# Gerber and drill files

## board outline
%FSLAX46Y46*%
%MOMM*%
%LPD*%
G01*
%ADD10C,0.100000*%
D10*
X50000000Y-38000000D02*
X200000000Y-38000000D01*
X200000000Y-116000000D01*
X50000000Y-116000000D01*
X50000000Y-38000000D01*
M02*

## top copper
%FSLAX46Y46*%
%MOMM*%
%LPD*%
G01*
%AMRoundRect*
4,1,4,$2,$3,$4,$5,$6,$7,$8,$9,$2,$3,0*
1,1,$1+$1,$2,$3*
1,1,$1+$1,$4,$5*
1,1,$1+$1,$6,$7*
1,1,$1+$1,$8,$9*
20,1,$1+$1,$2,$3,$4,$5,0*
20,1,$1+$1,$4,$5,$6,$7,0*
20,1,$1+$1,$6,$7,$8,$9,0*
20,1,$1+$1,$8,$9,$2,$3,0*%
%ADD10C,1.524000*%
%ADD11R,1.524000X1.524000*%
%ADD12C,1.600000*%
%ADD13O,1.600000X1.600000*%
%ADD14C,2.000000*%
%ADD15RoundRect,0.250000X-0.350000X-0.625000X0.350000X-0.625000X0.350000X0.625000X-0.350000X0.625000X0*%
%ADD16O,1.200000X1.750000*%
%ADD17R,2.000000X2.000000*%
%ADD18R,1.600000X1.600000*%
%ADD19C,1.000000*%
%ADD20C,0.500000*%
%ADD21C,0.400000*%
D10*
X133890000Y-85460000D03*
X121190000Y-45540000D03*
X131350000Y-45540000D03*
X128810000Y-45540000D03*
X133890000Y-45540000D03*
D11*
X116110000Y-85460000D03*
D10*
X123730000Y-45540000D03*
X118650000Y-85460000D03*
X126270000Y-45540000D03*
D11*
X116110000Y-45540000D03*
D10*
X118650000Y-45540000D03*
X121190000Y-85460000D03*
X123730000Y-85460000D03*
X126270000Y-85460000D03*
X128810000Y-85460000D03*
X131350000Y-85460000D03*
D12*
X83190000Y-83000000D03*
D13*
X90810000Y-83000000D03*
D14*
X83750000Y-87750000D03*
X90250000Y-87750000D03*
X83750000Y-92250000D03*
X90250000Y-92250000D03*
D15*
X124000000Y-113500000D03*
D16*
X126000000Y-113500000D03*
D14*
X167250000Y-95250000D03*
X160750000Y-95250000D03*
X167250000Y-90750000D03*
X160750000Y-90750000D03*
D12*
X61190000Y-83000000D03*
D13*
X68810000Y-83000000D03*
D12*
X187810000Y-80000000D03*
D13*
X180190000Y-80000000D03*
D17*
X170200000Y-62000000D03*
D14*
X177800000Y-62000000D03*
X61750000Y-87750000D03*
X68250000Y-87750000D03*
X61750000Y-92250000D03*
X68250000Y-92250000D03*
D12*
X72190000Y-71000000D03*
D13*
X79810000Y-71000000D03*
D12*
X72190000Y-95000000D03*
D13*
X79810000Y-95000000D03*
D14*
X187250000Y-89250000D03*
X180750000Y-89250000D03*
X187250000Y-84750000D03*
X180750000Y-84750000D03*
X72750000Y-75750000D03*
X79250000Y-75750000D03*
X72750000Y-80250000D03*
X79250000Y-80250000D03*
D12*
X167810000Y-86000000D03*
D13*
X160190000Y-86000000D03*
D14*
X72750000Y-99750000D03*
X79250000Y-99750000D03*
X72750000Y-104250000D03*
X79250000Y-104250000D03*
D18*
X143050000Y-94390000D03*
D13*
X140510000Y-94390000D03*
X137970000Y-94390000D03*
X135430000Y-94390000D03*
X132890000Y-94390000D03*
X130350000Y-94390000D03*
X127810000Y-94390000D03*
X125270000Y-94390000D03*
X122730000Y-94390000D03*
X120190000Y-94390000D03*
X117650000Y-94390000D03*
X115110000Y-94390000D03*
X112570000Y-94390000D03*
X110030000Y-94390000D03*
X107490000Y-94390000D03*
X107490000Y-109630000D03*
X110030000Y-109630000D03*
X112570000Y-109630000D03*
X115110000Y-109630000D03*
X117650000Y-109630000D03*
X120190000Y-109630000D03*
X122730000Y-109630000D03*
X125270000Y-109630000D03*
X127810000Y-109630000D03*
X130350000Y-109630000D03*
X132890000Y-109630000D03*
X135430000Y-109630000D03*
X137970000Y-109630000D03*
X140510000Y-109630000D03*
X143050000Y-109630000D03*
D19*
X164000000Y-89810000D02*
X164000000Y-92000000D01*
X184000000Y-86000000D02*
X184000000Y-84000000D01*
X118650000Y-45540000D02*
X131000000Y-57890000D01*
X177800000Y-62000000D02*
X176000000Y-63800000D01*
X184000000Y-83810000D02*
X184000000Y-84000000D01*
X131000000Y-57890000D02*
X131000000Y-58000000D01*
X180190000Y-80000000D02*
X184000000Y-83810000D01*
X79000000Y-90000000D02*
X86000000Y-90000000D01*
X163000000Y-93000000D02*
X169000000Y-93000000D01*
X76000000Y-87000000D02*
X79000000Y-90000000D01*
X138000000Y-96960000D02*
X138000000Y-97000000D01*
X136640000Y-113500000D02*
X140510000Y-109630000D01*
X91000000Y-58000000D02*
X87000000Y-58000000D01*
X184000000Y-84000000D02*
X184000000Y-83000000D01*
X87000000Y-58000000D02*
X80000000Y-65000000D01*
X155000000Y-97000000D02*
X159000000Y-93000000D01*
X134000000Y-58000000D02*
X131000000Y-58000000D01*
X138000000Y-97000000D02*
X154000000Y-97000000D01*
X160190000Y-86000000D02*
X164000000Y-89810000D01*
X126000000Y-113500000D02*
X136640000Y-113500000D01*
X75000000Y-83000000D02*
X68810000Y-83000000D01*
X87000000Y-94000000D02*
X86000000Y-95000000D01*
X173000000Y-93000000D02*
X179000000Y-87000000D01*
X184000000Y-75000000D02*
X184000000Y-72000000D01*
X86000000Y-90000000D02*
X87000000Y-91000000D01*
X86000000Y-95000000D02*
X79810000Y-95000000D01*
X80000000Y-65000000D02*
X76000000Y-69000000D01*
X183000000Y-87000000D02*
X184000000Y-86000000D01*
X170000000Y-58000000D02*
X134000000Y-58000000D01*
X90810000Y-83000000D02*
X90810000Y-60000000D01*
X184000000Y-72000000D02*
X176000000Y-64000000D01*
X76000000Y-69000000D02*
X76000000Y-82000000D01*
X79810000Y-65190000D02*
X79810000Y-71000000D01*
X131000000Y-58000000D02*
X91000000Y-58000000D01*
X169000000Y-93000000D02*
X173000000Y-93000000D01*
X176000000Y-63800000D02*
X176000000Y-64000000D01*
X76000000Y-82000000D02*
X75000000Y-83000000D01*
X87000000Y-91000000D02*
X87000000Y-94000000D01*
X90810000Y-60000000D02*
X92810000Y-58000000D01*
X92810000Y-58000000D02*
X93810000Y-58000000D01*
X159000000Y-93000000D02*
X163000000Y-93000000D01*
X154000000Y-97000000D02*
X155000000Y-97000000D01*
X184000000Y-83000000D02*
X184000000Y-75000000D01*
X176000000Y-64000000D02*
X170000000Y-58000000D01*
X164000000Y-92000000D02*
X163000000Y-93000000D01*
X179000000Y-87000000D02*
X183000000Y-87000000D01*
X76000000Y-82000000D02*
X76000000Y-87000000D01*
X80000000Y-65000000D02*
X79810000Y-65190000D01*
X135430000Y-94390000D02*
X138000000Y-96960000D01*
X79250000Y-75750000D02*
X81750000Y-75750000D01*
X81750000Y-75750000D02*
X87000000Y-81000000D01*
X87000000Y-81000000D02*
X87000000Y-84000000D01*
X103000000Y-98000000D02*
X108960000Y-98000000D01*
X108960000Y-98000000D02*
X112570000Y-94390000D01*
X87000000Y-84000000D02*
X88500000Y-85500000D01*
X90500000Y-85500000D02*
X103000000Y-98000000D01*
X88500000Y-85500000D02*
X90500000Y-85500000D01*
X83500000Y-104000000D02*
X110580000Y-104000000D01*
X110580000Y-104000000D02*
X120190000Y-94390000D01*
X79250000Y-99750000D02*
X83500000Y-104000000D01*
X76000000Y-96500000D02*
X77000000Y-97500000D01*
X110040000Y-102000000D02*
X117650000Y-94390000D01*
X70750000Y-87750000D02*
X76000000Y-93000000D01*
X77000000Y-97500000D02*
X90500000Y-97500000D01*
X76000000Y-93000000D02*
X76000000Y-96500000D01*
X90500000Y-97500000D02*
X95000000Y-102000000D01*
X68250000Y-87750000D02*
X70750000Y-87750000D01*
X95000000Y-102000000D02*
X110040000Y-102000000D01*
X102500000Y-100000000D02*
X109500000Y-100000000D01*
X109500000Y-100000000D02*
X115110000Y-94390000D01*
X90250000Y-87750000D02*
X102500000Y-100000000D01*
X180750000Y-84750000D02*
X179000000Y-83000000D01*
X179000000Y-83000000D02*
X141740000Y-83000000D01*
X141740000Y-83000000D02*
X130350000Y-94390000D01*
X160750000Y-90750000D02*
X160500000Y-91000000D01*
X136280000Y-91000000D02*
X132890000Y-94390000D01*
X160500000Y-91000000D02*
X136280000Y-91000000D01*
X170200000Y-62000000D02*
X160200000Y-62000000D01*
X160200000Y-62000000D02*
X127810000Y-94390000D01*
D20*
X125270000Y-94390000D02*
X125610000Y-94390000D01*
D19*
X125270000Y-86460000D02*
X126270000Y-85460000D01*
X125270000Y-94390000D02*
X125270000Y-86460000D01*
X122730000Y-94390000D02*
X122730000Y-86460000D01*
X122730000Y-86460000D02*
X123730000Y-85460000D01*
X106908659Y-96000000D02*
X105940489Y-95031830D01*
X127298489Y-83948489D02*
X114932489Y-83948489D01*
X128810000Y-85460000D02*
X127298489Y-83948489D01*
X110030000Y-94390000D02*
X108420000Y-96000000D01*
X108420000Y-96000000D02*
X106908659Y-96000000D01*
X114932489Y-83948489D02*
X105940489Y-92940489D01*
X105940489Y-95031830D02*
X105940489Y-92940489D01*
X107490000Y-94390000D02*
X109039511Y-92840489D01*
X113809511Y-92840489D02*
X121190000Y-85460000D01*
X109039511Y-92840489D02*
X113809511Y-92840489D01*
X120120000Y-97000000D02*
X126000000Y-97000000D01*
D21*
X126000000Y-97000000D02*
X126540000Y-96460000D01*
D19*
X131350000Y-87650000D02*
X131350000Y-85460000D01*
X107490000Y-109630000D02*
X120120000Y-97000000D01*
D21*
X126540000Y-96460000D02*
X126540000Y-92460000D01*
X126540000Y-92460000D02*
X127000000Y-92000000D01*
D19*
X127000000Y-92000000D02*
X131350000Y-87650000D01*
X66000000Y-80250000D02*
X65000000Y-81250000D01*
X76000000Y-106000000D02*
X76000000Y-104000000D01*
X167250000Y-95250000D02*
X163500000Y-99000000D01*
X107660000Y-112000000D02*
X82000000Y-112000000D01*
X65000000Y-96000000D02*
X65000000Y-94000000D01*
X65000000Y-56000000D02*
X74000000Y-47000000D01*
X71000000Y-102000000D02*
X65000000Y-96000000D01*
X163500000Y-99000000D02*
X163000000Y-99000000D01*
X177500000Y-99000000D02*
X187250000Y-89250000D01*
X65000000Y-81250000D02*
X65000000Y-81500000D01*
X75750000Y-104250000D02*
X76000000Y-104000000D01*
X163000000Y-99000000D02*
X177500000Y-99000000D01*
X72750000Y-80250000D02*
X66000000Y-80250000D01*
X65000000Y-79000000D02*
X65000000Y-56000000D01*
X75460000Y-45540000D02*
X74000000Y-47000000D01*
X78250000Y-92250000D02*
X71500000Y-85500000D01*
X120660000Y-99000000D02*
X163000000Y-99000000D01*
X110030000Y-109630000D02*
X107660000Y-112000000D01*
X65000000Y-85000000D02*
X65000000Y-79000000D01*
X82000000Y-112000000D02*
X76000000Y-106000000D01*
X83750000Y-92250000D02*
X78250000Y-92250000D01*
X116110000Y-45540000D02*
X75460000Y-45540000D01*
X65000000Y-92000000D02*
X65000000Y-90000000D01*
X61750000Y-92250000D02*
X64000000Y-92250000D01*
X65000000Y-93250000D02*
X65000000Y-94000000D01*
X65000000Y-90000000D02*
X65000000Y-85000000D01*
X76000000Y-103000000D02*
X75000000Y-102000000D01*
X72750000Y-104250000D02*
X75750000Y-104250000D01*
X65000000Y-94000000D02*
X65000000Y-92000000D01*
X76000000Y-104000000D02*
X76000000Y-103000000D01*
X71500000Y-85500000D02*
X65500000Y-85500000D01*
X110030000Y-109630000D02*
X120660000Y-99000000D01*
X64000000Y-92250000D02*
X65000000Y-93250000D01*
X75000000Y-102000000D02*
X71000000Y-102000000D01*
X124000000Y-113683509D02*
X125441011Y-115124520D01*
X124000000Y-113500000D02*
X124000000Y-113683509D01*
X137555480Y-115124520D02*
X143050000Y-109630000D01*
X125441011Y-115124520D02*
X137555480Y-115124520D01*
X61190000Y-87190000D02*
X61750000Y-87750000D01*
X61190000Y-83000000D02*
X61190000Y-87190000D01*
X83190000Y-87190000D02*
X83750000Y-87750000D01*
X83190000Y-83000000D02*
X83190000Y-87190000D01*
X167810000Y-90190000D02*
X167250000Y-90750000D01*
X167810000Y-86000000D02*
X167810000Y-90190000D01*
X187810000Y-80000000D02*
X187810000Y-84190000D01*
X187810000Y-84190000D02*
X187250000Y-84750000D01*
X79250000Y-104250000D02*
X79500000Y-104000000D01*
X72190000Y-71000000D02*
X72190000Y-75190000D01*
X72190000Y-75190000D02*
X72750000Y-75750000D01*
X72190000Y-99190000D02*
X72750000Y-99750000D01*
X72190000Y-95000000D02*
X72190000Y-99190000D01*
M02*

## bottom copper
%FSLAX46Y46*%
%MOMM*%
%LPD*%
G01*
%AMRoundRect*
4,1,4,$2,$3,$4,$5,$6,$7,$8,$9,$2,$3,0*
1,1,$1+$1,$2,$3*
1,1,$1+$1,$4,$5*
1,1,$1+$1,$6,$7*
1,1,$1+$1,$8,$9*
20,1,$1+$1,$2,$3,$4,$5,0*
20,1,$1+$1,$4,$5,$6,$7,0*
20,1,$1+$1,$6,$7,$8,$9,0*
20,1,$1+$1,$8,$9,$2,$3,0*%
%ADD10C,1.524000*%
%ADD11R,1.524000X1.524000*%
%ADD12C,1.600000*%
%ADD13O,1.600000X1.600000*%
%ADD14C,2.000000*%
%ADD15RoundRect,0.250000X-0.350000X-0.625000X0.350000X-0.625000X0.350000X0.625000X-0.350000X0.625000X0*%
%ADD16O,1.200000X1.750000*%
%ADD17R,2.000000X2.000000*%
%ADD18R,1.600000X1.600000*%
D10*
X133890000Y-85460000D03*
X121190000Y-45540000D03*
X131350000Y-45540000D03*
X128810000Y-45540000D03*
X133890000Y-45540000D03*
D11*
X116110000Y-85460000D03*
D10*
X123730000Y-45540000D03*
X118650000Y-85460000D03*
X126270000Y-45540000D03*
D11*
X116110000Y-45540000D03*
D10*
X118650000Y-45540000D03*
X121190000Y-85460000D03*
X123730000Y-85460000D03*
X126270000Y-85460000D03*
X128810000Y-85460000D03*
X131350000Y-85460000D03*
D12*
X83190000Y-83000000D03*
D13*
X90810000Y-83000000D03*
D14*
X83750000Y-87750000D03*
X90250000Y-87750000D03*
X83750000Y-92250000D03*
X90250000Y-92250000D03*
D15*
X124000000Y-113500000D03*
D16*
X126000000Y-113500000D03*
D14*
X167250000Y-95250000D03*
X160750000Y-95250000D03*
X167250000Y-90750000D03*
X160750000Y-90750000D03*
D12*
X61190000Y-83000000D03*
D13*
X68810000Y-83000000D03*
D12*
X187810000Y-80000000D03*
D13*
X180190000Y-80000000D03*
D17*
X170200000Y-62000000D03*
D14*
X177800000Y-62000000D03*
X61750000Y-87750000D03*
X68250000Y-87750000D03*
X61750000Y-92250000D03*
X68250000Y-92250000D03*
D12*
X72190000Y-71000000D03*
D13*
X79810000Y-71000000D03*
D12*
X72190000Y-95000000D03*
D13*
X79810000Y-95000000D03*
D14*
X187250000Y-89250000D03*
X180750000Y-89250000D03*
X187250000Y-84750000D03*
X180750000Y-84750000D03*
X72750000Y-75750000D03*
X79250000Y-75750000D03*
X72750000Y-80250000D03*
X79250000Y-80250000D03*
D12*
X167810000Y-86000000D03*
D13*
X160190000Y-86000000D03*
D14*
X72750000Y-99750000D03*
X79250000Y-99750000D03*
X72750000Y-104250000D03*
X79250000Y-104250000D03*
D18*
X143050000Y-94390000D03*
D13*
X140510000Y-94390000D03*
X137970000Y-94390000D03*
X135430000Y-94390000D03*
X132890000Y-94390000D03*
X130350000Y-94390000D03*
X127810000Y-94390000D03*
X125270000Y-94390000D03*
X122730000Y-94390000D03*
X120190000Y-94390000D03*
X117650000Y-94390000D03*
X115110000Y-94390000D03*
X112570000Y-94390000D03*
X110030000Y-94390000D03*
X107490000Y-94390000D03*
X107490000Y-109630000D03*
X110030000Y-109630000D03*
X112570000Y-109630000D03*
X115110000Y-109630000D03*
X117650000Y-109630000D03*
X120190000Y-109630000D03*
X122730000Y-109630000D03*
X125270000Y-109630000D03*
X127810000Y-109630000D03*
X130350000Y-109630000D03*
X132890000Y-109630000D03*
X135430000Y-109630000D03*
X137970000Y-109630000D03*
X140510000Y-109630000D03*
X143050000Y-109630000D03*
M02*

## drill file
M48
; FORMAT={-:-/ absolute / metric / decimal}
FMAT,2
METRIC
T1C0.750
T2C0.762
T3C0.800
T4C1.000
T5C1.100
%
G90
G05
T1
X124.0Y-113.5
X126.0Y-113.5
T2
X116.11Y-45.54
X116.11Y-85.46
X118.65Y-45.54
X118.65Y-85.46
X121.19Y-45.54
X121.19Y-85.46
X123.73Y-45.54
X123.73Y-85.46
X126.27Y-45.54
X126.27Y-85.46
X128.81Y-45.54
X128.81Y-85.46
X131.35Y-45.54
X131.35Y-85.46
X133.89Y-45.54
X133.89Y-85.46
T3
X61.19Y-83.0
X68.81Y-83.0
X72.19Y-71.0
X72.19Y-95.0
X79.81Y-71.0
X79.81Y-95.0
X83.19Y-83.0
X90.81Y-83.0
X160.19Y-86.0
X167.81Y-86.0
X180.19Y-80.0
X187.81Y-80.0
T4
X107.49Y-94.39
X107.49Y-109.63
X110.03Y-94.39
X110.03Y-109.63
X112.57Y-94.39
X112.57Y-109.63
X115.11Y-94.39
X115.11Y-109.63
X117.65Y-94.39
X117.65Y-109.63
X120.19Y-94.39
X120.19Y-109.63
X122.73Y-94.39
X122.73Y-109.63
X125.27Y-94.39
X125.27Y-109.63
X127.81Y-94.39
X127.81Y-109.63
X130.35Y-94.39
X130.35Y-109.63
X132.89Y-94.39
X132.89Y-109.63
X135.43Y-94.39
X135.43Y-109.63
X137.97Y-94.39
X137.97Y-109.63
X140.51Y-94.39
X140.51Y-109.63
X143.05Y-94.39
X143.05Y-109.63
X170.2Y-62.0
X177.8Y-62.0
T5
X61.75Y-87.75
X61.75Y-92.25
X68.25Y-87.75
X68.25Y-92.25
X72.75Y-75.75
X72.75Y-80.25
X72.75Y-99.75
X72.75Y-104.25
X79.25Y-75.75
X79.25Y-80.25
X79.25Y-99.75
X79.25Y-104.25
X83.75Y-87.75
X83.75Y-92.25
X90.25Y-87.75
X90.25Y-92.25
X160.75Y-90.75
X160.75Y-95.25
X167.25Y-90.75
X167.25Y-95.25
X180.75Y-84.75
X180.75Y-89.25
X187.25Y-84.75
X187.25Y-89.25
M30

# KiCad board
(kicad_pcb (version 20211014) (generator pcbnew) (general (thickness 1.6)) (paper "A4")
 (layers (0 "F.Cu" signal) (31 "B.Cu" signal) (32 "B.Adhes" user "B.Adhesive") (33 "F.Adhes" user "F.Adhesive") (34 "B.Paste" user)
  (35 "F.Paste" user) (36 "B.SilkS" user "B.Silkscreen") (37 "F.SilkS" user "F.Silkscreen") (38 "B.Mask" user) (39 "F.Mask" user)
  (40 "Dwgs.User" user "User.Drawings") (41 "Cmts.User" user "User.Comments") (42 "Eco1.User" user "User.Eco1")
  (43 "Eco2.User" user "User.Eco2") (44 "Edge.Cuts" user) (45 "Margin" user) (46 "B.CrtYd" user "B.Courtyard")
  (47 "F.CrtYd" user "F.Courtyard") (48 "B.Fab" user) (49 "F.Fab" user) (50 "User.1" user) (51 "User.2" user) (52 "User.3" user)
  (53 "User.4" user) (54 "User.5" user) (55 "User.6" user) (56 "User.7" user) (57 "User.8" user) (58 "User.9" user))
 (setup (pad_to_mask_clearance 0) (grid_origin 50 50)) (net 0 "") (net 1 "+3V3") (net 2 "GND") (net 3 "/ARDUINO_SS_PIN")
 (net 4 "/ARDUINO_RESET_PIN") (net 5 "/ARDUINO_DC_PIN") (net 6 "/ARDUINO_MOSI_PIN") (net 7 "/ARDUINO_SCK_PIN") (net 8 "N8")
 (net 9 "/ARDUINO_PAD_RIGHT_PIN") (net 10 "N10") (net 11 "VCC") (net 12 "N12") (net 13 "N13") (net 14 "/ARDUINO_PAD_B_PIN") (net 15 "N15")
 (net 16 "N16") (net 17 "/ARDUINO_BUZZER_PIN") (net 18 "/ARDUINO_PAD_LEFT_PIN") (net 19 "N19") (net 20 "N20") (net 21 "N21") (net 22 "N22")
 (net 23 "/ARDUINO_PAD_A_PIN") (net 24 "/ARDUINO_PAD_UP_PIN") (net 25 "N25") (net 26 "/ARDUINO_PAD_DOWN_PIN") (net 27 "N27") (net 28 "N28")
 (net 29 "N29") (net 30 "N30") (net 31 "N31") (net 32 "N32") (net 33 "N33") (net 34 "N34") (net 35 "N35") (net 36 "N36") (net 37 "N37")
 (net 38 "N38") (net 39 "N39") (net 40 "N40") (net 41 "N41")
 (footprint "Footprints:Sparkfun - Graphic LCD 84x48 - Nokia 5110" (layer "F.Cu") (at 125 43)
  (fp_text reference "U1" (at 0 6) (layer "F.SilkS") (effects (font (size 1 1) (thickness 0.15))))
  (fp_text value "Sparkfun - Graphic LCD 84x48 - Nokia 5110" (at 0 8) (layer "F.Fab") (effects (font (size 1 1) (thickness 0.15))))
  (pad "" thru_hole circle (at 8.89 42.46) (size 1.524 1.524) (drill 0.762) (layers *.Cu *.Mask))
  (pad "" thru_hole circle (at -3.81 2.54) (size 1.524 1.524) (drill 0.762) (layers *.Cu *.Mask))
  (pad "" thru_hole circle (at 6.35 2.54) (size 1.524 1.524) (drill 0.762) (layers *.Cu *.Mask))
  (pad "" thru_hole circle (at 3.81 2.54) (size 1.524 1.524) (drill 0.762) (layers *.Cu *.Mask))
  (pad "" thru_hole circle (at 8.89 2.54) (size 1.524 1.524) (drill 0.762) (layers *.Cu *.Mask))
  (pad "" thru_hole rect (at -8.89 42.46) (size 1.524 1.524) (drill 0.762) (layers *.Cu *.Mask))
  (pad "" thru_hole circle (at -1.27 2.54) (size 1.524 1.524) (drill 0.762) (layers *.Cu *.Mask))
  (pad "" thru_hole circle (at -6.35 42.46) (size 1.524 1.524) (drill 0.762) (layers *.Cu *.Mask))
  (pad "" thru_hole circle (at 1.27 2.54) (size 1.524 1.524) (drill 0.762) (layers *.Cu *.Mask))
  (pad "1" thru_hole rect (at -8.89 2.54) (size 1.524 1.524) (drill 0.762) (layers *.Cu *.Mask) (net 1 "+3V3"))
  (pad "2" thru_hole circle (at -6.35 2.54) (size 1.524 1.524) (drill 0.762) (layers *.Cu *.Mask) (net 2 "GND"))
  (pad "3" thru_hole circle (at -3.81 42.46) (size 1.524 1.524) (drill 0.762) (layers *.Cu *.Mask) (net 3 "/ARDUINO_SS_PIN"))
  (pad "4" thru_hole circle (at -1.27 42.46) (size 1.524 1.524) (drill 0.762) (layers *.Cu *.Mask) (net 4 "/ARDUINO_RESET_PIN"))
  (pad "5" thru_hole circle (at 1.27 42.46) (size 1.524 1.524) (drill 0.762) (layers *.Cu *.Mask) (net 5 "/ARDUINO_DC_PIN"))
  (pad "6" thru_hole circle (at 3.81 42.46) (size 1.524 1.524) (drill 0.762) (layers *.Cu *.Mask) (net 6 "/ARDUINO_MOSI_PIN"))
  (pad "7" thru_hole circle (at 6.35 42.46) (size 1.524 1.524) (drill 0.762) (layers *.Cu *.Mask) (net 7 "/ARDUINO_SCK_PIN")))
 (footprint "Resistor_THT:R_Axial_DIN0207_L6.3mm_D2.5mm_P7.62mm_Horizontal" (layer "F.Cu") (at 83.19 83)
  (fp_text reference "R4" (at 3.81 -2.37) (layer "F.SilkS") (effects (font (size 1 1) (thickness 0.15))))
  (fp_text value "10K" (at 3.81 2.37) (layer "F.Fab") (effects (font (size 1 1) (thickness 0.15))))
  (pad "1" thru_hole circle (at 0 0) (size 1.6 1.6) (drill 0.8) (layers *.Cu *.Mask) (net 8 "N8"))
  (pad "2" thru_hole oval (at 7.62 0) (size 1.6 1.6) (drill 0.8) (layers *.Cu *.Mask) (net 2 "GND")))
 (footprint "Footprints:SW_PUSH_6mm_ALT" (layer "F.Cu") (at 83.75 87.75)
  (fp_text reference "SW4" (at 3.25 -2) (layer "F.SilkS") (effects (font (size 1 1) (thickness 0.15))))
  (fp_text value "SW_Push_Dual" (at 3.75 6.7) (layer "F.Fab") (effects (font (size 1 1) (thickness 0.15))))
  (pad "1" thru_hole circle (at 0 0 90) (size 2 2) (drill 1.1) (layers *.Cu *.Mask) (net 8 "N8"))
  (pad "2" thru_hole circle (at 6.5 0 90) (size 2 2) (drill 1.1) (layers *.Cu *.Mask) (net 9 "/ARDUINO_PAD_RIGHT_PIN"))
  (pad "3" thru_hole circle (at 0 4.5 90) (size 2 2) (drill 1.1) (layers *.Cu *.Mask) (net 1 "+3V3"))
  (pad "4" thru_hole circle (at 6.5 4.5 90) (size 2 2) (drill 1.1) (layers *.Cu *.Mask) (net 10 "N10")))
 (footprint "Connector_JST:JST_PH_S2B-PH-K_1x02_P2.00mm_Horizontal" (layer "F.Cu") (at 124 113.5)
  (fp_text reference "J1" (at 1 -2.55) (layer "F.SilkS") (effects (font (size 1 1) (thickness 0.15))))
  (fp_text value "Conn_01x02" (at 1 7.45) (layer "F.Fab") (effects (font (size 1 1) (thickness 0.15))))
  (pad "1" thru_hole roundrect (at 0 0) (size 1.2 1.75) (drill 0.75) (layers *.Cu *.Mask) (roundrect_rratio 0.208333) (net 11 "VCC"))
  (pad "2" thru_hole oval (at 2 0) (size 1.2 1.75) (drill 0.75) (layers *.Cu *.Mask) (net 2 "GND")))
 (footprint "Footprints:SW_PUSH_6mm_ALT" (layer "F.Cu") (at 167.25 95.25 180)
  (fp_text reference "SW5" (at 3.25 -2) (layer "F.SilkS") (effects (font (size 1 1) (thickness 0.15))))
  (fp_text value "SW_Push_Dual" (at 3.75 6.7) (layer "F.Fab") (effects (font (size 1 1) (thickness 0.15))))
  (pad "1" thru_hole circle (at 0 0 270) (size 2 2) (drill 1.1) (layers *.Cu *.Mask) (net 1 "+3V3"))
  (pad "2" thru_hole circle (at 6.5 0 270) (size 2 2) (drill 1.1) (layers *.Cu *.Mask) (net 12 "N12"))
  (pad "3" thru_hole circle (at 0 4.5 270) (size 2 2) (drill 1.1) (layers *.Cu *.Mask) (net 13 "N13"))
  (pad "4" thru_hole circle (at 6.5 4.5 270) (size 2 2) (drill 1.1) (layers *.Cu *.Mask) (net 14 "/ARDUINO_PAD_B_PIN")))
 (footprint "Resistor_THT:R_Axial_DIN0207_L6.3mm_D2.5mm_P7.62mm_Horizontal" (layer "F.Cu") (at 61.19 83)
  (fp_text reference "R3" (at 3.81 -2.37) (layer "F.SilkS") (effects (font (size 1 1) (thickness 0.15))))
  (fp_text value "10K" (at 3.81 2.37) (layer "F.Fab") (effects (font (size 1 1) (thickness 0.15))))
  (pad "1" thru_hole circle (at 0 0) (size 1.6 1.6) (drill 0.8) (layers *.Cu *.Mask) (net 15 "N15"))
  (pad "2" thru_hole oval (at 7.62 0) (size 1.6 1.6) (drill 0.8) (layers *.Cu *.Mask) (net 2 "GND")))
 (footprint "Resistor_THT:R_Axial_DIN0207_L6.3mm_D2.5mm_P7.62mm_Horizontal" (layer "F.Cu") (at 187.81 80 180)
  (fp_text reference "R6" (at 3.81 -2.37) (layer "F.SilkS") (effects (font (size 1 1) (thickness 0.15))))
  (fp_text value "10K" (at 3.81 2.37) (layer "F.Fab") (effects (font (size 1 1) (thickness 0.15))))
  (pad "1" thru_hole circle (at 0 0 180) (size 1.6 1.6) (drill 0.8) (layers *.Cu *.Mask) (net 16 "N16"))
  (pad "2" thru_hole oval (at 7.62 0 180) (size 1.6 1.6) (drill 0.8) (layers *.Cu *.Mask) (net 2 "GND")))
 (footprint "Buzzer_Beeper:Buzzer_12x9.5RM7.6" (layer "F.Cu") (at 170.2 62)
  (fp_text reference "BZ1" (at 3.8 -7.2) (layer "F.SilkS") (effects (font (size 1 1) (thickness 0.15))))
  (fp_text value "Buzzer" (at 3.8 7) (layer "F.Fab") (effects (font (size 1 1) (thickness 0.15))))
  (pad "1" thru_hole rect (at 0 0) (size 2 2) (drill 1) (layers *.Cu *.Mask) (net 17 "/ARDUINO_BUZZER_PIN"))
  (pad "2" thru_hole circle (at 7.6 0) (size 2 2) (drill 1) (layers *.Cu *.Mask) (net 2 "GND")))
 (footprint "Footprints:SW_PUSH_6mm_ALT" (layer "F.Cu") (at 61.75 87.75)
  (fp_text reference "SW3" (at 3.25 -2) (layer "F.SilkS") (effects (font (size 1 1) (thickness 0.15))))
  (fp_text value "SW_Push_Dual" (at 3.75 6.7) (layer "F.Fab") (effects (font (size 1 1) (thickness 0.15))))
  (pad "1" thru_hole circle (at 0 0 90) (size 2 2) (drill 1.1) (layers *.Cu *.Mask) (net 15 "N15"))
  (pad "2" thru_hole circle (at 6.5 0 90) (size 2 2) (drill 1.1) (layers *.Cu *.Mask) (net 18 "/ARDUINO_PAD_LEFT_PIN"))
  (pad "3" thru_hole circle (at 0 4.5 90) (size 2 2) (drill 1.1) (layers *.Cu *.Mask) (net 1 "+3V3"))
  (pad "4" thru_hole circle (at 6.5 4.5 90) (size 2 2) (drill 1.1) (layers *.Cu *.Mask) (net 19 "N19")))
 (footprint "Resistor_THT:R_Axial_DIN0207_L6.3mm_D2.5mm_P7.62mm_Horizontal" (layer "F.Cu") (at 72.19 71)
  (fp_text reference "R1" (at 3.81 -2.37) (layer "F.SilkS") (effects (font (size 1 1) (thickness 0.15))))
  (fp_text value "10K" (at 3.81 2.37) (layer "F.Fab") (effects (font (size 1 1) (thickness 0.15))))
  (pad "1" thru_hole circle (at 0 0) (size 1.6 1.6) (drill 0.8) (layers *.Cu *.Mask) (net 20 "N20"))
  (pad "2" thru_hole oval (at 7.62 0) (size 1.6 1.6) (drill 0.8) (layers *.Cu *.Mask) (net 2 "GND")))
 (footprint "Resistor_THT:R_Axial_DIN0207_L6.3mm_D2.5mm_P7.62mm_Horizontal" (layer "F.Cu") (at 72.19 95)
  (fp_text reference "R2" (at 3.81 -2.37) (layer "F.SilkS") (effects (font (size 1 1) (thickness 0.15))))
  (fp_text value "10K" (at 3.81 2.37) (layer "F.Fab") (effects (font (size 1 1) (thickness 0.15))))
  (pad "1" thru_hole circle (at 0 0) (size 1.6 1.6) (drill 0.8) (layers *.Cu *.Mask) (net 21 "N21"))
  (pad "2" thru_hole oval (at 7.62 0) (size 1.6 1.6) (drill 0.8) (layers *.Cu *.Mask) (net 2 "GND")))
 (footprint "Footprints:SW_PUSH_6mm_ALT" (layer "F.Cu") (at 187.25 89.25 180)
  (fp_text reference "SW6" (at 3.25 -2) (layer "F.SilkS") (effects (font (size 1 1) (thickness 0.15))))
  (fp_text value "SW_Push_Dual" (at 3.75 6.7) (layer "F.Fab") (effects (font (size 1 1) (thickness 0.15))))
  (pad "1" thru_hole circle (at 0 0 270) (size 2 2) (drill 1.1) (layers *.Cu *.Mask) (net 1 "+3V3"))
  (pad "2" thru_hole circle (at 6.5 0 270) (size 2 2) (drill 1.1) (layers *.Cu *.Mask) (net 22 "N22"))
  (pad "3" thru_hole circle (at 0 4.5 270) (size 2 2) (drill 1.1) (layers *.Cu *.Mask) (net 16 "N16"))
  (pad "4" thru_hole circle (at 6.5 4.5 270) (size 2 2) (drill 1.1) (layers *.Cu *.Mask) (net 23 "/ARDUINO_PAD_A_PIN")))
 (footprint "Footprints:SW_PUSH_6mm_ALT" (layer "F.Cu") (at 72.75 75.75)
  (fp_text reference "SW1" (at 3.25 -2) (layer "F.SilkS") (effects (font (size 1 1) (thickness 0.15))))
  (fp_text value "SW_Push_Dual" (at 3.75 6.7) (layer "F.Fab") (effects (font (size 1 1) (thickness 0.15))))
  (pad "1" thru_hole circle (at 0 0 90) (size 2 2) (drill 1.1) (layers *.Cu *.Mask) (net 20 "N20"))
  (pad "2" thru_hole circle (at 6.5 0 90) (size 2 2) (drill 1.1) (layers *.Cu *.Mask) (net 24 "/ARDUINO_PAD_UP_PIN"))
  (pad "3" thru_hole circle (at 0 4.5 90) (size 2 2) (drill 1.1) (layers *.Cu *.Mask) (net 1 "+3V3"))
  (pad "4" thru_hole circle (at 6.5 4.5 90) (size 2 2) (drill 1.1) (layers *.Cu *.Mask) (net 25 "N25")))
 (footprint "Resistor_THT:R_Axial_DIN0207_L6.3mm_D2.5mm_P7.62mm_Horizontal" (layer "F.Cu") (at 167.81 86 180)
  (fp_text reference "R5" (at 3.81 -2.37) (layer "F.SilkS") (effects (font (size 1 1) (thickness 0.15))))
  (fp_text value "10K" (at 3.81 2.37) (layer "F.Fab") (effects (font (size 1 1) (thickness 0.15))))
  (pad "1" thru_hole circle (at 0 0 180) (size 1.6 1.6) (drill 0.8) (layers *.Cu *.Mask) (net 13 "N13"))
  (pad "2" thru_hole oval (at 7.62 0 180) (size 1.6 1.6) (drill 0.8) (layers *.Cu *.Mask) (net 2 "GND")))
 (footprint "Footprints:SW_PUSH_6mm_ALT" (layer "F.Cu") (at 72.75 99.75)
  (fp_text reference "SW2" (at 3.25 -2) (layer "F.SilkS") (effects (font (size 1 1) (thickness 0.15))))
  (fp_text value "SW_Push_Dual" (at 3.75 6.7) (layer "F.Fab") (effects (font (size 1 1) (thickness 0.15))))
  (pad "1" thru_hole circle (at 0 0 90) (size 2 2) (drill 1.1) (layers *.Cu *.Mask) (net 21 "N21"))
  (pad "2" thru_hole circle (at 6.5 0 90) (size 2 2) (drill 1.1) (layers *.Cu *.Mask) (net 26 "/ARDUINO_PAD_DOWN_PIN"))
  (pad "3" thru_hole circle (at 0 4.5 90) (size 2 2) (drill 1.1) (layers *.Cu *.Mask) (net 1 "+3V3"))
  (pad "4" thru_hole circle (at 6.5 4.5 90) (size 2 2) (drill 1.1) (layers *.Cu *.Mask) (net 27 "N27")))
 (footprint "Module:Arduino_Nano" (layer "F.Cu") (at 143.05 94.39 -90)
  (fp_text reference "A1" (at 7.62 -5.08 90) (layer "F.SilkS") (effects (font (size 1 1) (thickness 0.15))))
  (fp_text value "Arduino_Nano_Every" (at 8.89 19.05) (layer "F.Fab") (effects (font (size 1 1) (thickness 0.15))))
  (pad "1" thru_hole rect (at 0 0 270) (size 1.6 1.6) (drill 1) (layers *.Cu *.Mask) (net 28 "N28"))
  (pad "2" thru_hole oval (at 0 2.54 270) (size 1.6 1.6) (drill 1) (layers *.Cu *.Mask) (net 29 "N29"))
  (pad "3" thru_hole oval (at 0 5.08 270) (size 1.6 1.6) (drill 1) (layers *.Cu *.Mask) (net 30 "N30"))
  (pad "4" thru_hole oval (at 0 7.62 270) (size 1.6 1.6) (drill 1) (layers *.Cu *.Mask) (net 2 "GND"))
  (pad "5" thru_hole oval (at 0 10.16 270) (size 1.6 1.6) (drill 1) (layers *.Cu *.Mask) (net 14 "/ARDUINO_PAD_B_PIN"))
  (pad "6" thru_hole oval (at 0 12.7 270) (size 1.6 1.6) (drill 1) (layers *.Cu *.Mask) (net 23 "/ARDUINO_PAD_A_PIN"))
  (pad "7" thru_hole oval (at 0 15.24 270) (size 1.6 1.6) (drill 1) (layers *.Cu *.Mask) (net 17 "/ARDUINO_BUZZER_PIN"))
  (pad "8" thru_hole oval (at 0 17.78 270) (size 1.6 1.6) (drill 1) (layers *.Cu *.Mask) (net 5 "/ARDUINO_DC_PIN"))
  (pad "9" thru_hole oval (at 0 20.32 270) (size 1.6 1.6) (drill 1) (layers *.Cu *.Mask) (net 4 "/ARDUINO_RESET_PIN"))
  (pad "10" thru_hole oval (at 0 22.86 270) (size 1.6 1.6) (drill 1) (layers *.Cu *.Mask) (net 26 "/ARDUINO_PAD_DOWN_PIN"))
  (pad "11" thru_hole oval (at 0 25.4 270) (size 1.6 1.6) (drill 1) (layers *.Cu *.Mask) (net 18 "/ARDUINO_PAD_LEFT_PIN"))
  (pad "12" thru_hole oval (at 0 27.94 270) (size 1.6 1.6) (drill 1) (layers *.Cu *.Mask) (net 9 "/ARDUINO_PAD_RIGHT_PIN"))
  (pad "13" thru_hole oval (at 0 30.48 270) (size 1.6 1.6) (drill 1) (layers *.Cu *.Mask) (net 24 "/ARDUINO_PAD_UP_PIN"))
  (pad "14" thru_hole oval (at 0 33.02 270) (size 1.6 1.6) (drill 1) (layers *.Cu *.Mask) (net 6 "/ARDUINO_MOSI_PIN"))
  (pad "15" thru_hole oval (at 0 35.56 270) (size 1.6 1.6) (drill 1) (layers *.Cu *.Mask) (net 3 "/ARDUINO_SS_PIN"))
  (pad "16" thru_hole oval (at 15.24 35.56 270) (size 1.6 1.6) (drill 1) (layers *.Cu *.Mask) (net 7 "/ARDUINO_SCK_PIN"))
  (pad "17" thru_hole oval (at 15.24 33.02 270) (size 1.6 1.6) (drill 1) (layers *.Cu *.Mask) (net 1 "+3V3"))
  (pad "18" thru_hole oval (at 15.24 30.48 270) (size 1.6 1.6) (drill 1) (layers *.Cu *.Mask) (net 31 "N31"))
  (pad "19" thru_hole oval (at 15.24 27.94 270) (size 1.6 1.6) (drill 1) (layers *.Cu *.Mask) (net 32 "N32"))
  (pad "20" thru_hole oval (at 15.24 25.4 270) (size 1.6 1.6) (drill 1) (layers *.Cu *.Mask) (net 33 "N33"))
  (pad "21" thru_hole oval (at 15.24 22.86 270) (size 1.6 1.6) (drill 1) (layers *.Cu *.Mask) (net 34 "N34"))
  (pad "22" thru_hole oval (at 15.24 20.32 270) (size 1.6 1.6) (drill 1) (layers *.Cu *.Mask) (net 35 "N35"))
  (pad "23" thru_hole oval (at 15.24 17.78 270) (size 1.6 1.6) (drill 1) (layers *.Cu *.Mask) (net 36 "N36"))
  (pad "24" thru_hole oval (at 15.24 15.24 270) (size 1.6 1.6) (drill 1) (layers *.Cu *.Mask) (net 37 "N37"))
  (pad "25" thru_hole oval (at 15.24 12.7 270) (size 1.6 1.6) (drill 1) (layers *.Cu *.Mask) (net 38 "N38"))
  (pad "26" thru_hole oval (at 15.24 10.16 270) (size 1.6 1.6) (drill 1) (layers *.Cu *.Mask) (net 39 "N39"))
  (pad "27" thru_hole oval (at 15.24 7.62 270) (size 1.6 1.6) (drill 1) (layers *.Cu *.Mask) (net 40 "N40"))
  (pad "28" thru_hole oval (at 15.24 5.08 270) (size 1.6 1.6) (drill 1) (layers *.Cu *.Mask) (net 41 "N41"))
  (pad "29" thru_hole oval (at 15.24 2.54 270) (size 1.6 1.6) (drill 1) (layers *.Cu *.Mask) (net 2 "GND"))
  (pad "30" thru_hole oval (at 15.24 0 270) (size 1.6 1.6) (drill 1) (layers *.Cu *.Mask) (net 11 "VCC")))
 (gr_rect (start 50 38) (end 200 116) (layer "Edge.Cuts") (width 0.1) (fill none))
 (segment (start 164 89.81) (end 164 92) (width 1) (layer "F.Cu") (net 2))
 (segment (start 184 86) (end 184 84) (width 1) (layer "F.Cu") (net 2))
 (segment (start 118.65 45.54) (end 131 57.89) (width 1) (layer "F.Cu") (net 2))
 (segment (start 177.8 62) (end 176 63.8) (width 1) (layer "F.Cu") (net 2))
 (segment (start 184 83.81) (end 184 84) (width 1) (layer "F.Cu") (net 2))
 (segment (start 131 57.89) (end 131 58) (width 1) (layer "F.Cu") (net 2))
 (segment (start 180.19 80) (end 184 83.81) (width 1) (layer "F.Cu") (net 2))
 (segment (start 79 90) (end 86 90) (width 1) (layer "F.Cu") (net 2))
 (segment (start 163 93) (end 169 93) (width 1) (layer "F.Cu") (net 2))
 (segment (start 76 87) (end 79 90) (width 1) (layer "F.Cu") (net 2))
 (segment (start 138 96.96) (end 138 97) (width 1) (layer "F.Cu") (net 2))
 (segment (start 136.64 113.5) (end 140.51 109.63) (width 1) (layer "F.Cu") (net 2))
 (segment (start 91 58) (end 87 58) (width 1) (layer "F.Cu") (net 2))
 (segment (start 184 84) (end 184 83) (width 1) (layer "F.Cu") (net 2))
 (segment (start 87 58) (end 80 65) (width 1) (layer "F.Cu") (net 2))
 (segment (start 155 97) (end 159 93) (width 1) (layer "F.Cu") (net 2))
 (segment (start 134 58) (end 131 58) (width 1) (layer "F.Cu") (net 2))
 (segment (start 138 97) (end 154 97) (width 1) (layer "F.Cu") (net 2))
 (segment (start 160.19 86) (end 164 89.81) (width 1) (layer "F.Cu") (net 2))
 (segment (start 126 113.5) (end 136.64 113.5) (width 1) (layer "F.Cu") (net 2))
 (segment (start 75 83) (end 68.81 83) (width 1) (layer "F.Cu") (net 2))
 (segment (start 87 94) (end 86 95) (width 1) (layer "F.Cu") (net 2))
 (segment (start 173 93) (end 179 87) (width 1) (layer "F.Cu") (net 2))
 (segment (start 184 75) (end 184 72) (width 1) (layer "F.Cu") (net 2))
 (segment (start 86 90) (end 87 91) (width 1) (layer "F.Cu") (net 2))
 (segment (start 86 95) (end 79.81 95) (width 1) (layer "F.Cu") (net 2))
 (segment (start 80 65) (end 76 69) (width 1) (layer "F.Cu") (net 2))
 (segment (start 183 87) (end 184 86) (width 1) (layer "F.Cu") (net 2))
 (segment (start 170 58) (end 134 58) (width 1) (layer "F.Cu") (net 2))
 (segment (start 90.81 83) (end 90.81 60) (width 1) (layer "F.Cu") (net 2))
 (segment (start 184 72) (end 176 64) (width 1) (layer "F.Cu") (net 2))
 (segment (start 76 69) (end 76 82) (width 1) (layer "F.Cu") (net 2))
 (segment (start 79.81 65.19) (end 79.81 71) (width 1) (layer "F.Cu") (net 2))
 (segment (start 131 58) (end 91 58) (width 1) (layer "F.Cu") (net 2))
 (segment (start 169 93) (end 173 93) (width 1) (layer "F.Cu") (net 2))
 (segment (start 176 63.8) (end 176 64) (width 1) (layer "F.Cu") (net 2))
 (segment (start 76 82) (end 75 83) (width 1) (layer "F.Cu") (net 2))
 (segment (start 87 91) (end 87 94) (width 1) (layer "F.Cu") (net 2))
 (segment (start 90.81 60) (end 92.81 58) (width 1) (layer "F.Cu") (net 2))
 (segment (start 92.81 58) (end 93.81 58) (width 1) (layer "F.Cu") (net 2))
 (segment (start 159 93) (end 163 93) (width 1) (layer "F.Cu") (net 2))
 (segment (start 154 97) (end 155 97) (width 1) (layer "F.Cu") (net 2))
 (segment (start 184 83) (end 184 75) (width 1) (layer "F.Cu") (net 2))
 (segment (start 176 64) (end 170 58) (width 1) (layer "F.Cu") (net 2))
 (segment (start 164 92) (end 163 93) (width 1) (layer "F.Cu") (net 2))
 (segment (start 179 87) (end 183 87) (width 1) (layer "F.Cu") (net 2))
 (segment (start 76 82) (end 76 87) (width 1) (layer "F.Cu") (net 2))
 (segment (start 80 65) (end 79.81 65.19) (width 1) (layer "F.Cu") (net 2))
 (segment (start 135.43 94.39) (end 138 96.96) (width 1) (layer "F.Cu") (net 2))
 (segment (start 79.25 75.75) (end 81.75 75.75) (width 1) (layer "F.Cu") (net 24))
 (segment (start 81.75 75.75) (end 87 81) (width 1) (layer "F.Cu") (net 24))
 (segment (start 87 81) (end 87 84) (width 1) (layer "F.Cu") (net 24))
 (segment (start 103 98) (end 108.96 98) (width 1) (layer "F.Cu") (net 24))
 (segment (start 108.96 98) (end 112.57 94.39) (width 1) (layer "F.Cu") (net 24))
 (segment (start 87 84) (end 88.5 85.5) (width 1) (layer "F.Cu") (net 24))
 (segment (start 90.5 85.5) (end 103 98) (width 1) (layer "F.Cu") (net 24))
 (segment (start 88.5 85.5) (end 90.5 85.5) (width 1) (layer "F.Cu") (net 24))
 (segment (start 83.5 104) (end 110.58 104) (width 1) (layer "F.Cu") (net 26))
 (segment (start 110.58 104) (end 120.19 94.39) (width 1) (layer "F.Cu") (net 26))
 (segment (start 79.25 99.75) (end 83.5 104) (width 1) (layer "F.Cu") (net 26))
 (segment (start 76 96.5) (end 77 97.5) (width 1) (layer "F.Cu") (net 18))
 (segment (start 110.04 102) (end 117.65 94.39) (width 1) (layer "F.Cu") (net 18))
 (segment (start 70.75 87.75) (end 76 93) (width 1) (layer "F.Cu") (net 18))
 (segment (start 77 97.5) (end 90.5 97.5) (width 1) (layer "F.Cu") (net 18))
 (segment (start 76 93) (end 76 96.5) (width 1) (layer "F.Cu") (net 18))
 (segment (start 90.5 97.5) (end 95 102) (width 1) (layer "F.Cu") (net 18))
 (segment (start 68.25 87.75) (end 70.75 87.75) (width 1) (layer "F.Cu") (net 18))
 (segment (start 95 102) (end 110.04 102) (width 1) (layer "F.Cu") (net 18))
 (segment (start 102.5 100) (end 109.5 100) (width 1) (layer "F.Cu") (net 9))
 (segment (start 109.5 100) (end 115.11 94.39) (width 1) (layer "F.Cu") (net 9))
 (segment (start 90.25 87.75) (end 102.5 100) (width 1) (layer "F.Cu") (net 9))
 (segment (start 180.75 84.75) (end 179 83) (width 1) (layer "F.Cu") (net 23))
 (segment (start 179 83) (end 141.74 83) (width 1) (layer "F.Cu") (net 23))
 (segment (start 141.74 83) (end 130.35 94.39) (width 1) (layer "F.Cu") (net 23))
 (segment (start 160.75 90.75) (end 160.5 91) (width 1) (layer "F.Cu") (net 14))
 (segment (start 136.28 91) (end 132.89 94.39) (width 1) (layer "F.Cu") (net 14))
 (segment (start 160.5 91) (end 136.28 91) (width 1) (layer "F.Cu") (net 14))
 (segment (start 170.2 62) (end 160.2 62) (width 1) (layer "F.Cu") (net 17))
 (segment (start 160.2 62) (end 127.81 94.39) (width 1) (layer "F.Cu") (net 17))
 (segment (start 125.27 94.39) (end 125.61 94.39) (width 0.5) (layer "F.Cu") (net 5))
 (segment (start 125.27 86.46) (end 126.27 85.46) (width 1) (layer "F.Cu") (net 5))
 (segment (start 125.27 94.39) (end 125.27 86.46) (width 1) (layer "F.Cu") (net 5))
 (segment (start 122.73 94.39) (end 122.73 86.46) (width 1) (layer "F.Cu") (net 4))
 (segment (start 122.73 86.46) (end 123.73 85.46) (width 1) (layer "F.Cu") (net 4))
 (segment (start 106.908659 96) (end 105.940489 95.03183) (width 1) (layer "F.Cu") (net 6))
 (segment (start 127.298489 83.948489) (end 114.932489 83.948489) (width 1) (layer "F.Cu") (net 6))
 (segment (start 128.81 85.46) (end 127.298489 83.948489) (width 1) (layer "F.Cu") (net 6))
 (segment (start 110.03 94.39) (end 108.42 96) (width 1) (layer "F.Cu") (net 6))
 (segment (start 108.42 96) (end 106.908659 96) (width 1) (layer "F.Cu") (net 6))
 (segment (start 114.932489 83.948489) (end 105.940489 92.940489) (width 1) (layer "F.Cu") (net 6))
 (segment (start 105.940489 95.03183) (end 105.940489 92.940489) (width 1) (layer "F.Cu") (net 6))
 (segment (start 107.49 94.39) (end 109.039511 92.840489) (width 1) (layer "F.Cu") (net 3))
 (segment (start 113.809511 92.840489) (end 121.19 85.46) (width 1) (layer "F.Cu") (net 3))
 (segment (start 109.039511 92.840489) (end 113.809511 92.840489) (width 1) (layer "F.Cu") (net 3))
 (segment (start 120.12 97) (end 126 97) (width 1) (layer "F.Cu") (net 7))
 (segment (start 126 97) (end 126.54 96.46) (width 0.4) (layer "F.Cu") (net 7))
 (segment (start 131.35 87.65) (end 131.35 85.46) (width 1) (layer "F.Cu") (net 7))
 (segment (start 107.49 109.63) (end 120.12 97) (width 1) (layer "F.Cu") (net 7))
 (segment (start 126.54 96.46) (end 126.54 92.46) (width 0.4) (layer "F.Cu") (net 7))
 (segment (start 126.54 92.46) (end 127 92) (width 0.4) (layer "F.Cu") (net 7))
 (segment (start 127 92) (end 131.35 87.65) (width 1) (layer "F.Cu") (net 7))
 (segment (start 66 80.25) (end 65 81.25) (width 1) (layer "F.Cu") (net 1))
 (segment (start 76 106) (end 76 104) (width 1) (layer "F.Cu") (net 1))
 (segment (start 167.25 95.25) (end 163.5 99) (width 1) (layer "F.Cu") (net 1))
 (segment (start 107.66 112) (end 82 112) (width 1) (layer "F.Cu") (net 1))
 (segment (start 65 96) (end 65 94) (width 1) (layer "F.Cu") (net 1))
 (segment (start 65 56) (end 74 47) (width 1) (layer "F.Cu") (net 1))
 (segment (start 71 102) (end 65 96) (width 1) (layer "F.Cu") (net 1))
 (segment (start 163.5 99) (end 163 99) (width 1) (layer "F.Cu") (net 1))
 (segment (start 177.5 99) (end 187.25 89.25) (width 1) (layer "F.Cu") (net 1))
 (segment (start 65 81.25) (end 65 81.5) (width 1) (layer "F.Cu") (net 1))
 (segment (start 75.75 104.25) (end 76 104) (width 1) (layer "F.Cu") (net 1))
 (segment (start 163 99) (end 177.5 99) (width 1) (layer "F.Cu") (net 1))
 (segment (start 72.75 80.25) (end 66 80.25) (width 1) (layer "F.Cu") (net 1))
 (segment (start 65 79) (end 65 56) (width 1) (layer "F.Cu") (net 1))
 (segment (start 75.46 45.54) (end 74 47) (width 1) (layer "F.Cu") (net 1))
 (segment (start 78.25 92.25) (end 71.5 85.5) (width 1) (layer "F.Cu") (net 1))
 (segment (start 120.66 99) (end 163 99) (width 1) (layer "F.Cu") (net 1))
 (segment (start 110.03 109.63) (end 107.66 112) (width 1) (layer "F.Cu") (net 1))
 (segment (start 65 85) (end 65 79) (width 1) (layer "F.Cu") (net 1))
 (segment (start 82 112) (end 76 106) (width 1) (layer "F.Cu") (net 1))
 (segment (start 83.75 92.25) (end 78.25 92.25) (width 1) (layer "F.Cu") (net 1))
 (segment (start 116.11 45.54) (end 75.46 45.54) (width 1) (layer "F.Cu") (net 1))
 (segment (start 65 92) (end 65 90) (width 1) (layer "F.Cu") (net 1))
 (segment (start 61.75 92.25) (end 64 92.25) (width 1) (layer "F.Cu") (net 1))
 (segment (start 65 93.25) (end 65 94) (width 1) (layer "F.Cu") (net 1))
 (segment (start 65 90) (end 65 85) (width 1) (layer "F.Cu") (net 1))
 (segment (start 76 103) (end 75 102) (width 1) (layer "F.Cu") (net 1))
 (segment (start 72.75 104.25) (end 75.75 104.25) (width 1) (layer "F.Cu") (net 1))
 (segment (start 65 94) (end 65 92) (width 1) (layer "F.Cu") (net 1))
 (segment (start 76 104) (end 76 103) (width 1) (layer "F.Cu") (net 1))
 (segment (start 71.5 85.5) (end 65.5 85.5) (width 1) (layer "F.Cu") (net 1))
 (segment (start 110.03 109.63) (end 120.66 99) (width 1) (layer "F.Cu") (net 1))
 (segment (start 64 92.25) (end 65 93.25) (width 1) (layer "F.Cu") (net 1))
 (segment (start 75 102) (end 71 102) (width 1) (layer "F.Cu") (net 1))
 (segment (start 124 113.683509) (end 125.441011 115.12452) (width 1) (layer "F.Cu") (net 11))
 (segment (start 124 113.5) (end 124 113.683509) (width 1) (layer "F.Cu") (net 11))
 (segment (start 137.55548 115.12452) (end 143.05 109.63) (width 1) (layer "F.Cu") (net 11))
 (segment (start 125.441011 115.12452) (end 137.55548 115.12452) (width 1) (layer "F.Cu") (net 11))
 (segment (start 61.19 87.19) (end 61.75 87.75) (width 1) (layer "F.Cu") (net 15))
 (segment (start 61.19 83) (end 61.19 87.19) (width 1) (layer "F.Cu") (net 15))
 (segment (start 83.19 87.19) (end 83.75 87.75) (width 1) (layer "F.Cu") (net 8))
 (segment (start 83.19 83) (end 83.19 87.19) (width 1) (layer "F.Cu") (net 8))
 (segment (start 167.81 90.19) (end 167.25 90.75) (width 1) (layer "F.Cu") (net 13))
 (segment (start 167.81 86) (end 167.81 90.19) (width 1) (layer "F.Cu") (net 13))
 (segment (start 187.81 80) (end 187.81 84.19) (width 1) (layer "F.Cu") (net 16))
 (segment (start 187.81 84.19) (end 187.25 84.75) (width 1) (layer "F.Cu") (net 16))
 (segment (start 79.25 104.25) (end 79.5 104) (width 1) (layer "F.Cu") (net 27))
 (segment (start 72.19 71) (end 72.19 75.19) (width 1) (layer "F.Cu") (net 20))
 (segment (start 72.19 75.19) (end 72.75 75.75) (width 1) (layer "F.Cu") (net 20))
 (segment (start 72.19 99.19) (end 72.75 99.75) (width 1) (layer "F.Cu") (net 21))
 (segment (start 72.19 95) (end 72.19 99.19) (width 1) (layer "F.Cu") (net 21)))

